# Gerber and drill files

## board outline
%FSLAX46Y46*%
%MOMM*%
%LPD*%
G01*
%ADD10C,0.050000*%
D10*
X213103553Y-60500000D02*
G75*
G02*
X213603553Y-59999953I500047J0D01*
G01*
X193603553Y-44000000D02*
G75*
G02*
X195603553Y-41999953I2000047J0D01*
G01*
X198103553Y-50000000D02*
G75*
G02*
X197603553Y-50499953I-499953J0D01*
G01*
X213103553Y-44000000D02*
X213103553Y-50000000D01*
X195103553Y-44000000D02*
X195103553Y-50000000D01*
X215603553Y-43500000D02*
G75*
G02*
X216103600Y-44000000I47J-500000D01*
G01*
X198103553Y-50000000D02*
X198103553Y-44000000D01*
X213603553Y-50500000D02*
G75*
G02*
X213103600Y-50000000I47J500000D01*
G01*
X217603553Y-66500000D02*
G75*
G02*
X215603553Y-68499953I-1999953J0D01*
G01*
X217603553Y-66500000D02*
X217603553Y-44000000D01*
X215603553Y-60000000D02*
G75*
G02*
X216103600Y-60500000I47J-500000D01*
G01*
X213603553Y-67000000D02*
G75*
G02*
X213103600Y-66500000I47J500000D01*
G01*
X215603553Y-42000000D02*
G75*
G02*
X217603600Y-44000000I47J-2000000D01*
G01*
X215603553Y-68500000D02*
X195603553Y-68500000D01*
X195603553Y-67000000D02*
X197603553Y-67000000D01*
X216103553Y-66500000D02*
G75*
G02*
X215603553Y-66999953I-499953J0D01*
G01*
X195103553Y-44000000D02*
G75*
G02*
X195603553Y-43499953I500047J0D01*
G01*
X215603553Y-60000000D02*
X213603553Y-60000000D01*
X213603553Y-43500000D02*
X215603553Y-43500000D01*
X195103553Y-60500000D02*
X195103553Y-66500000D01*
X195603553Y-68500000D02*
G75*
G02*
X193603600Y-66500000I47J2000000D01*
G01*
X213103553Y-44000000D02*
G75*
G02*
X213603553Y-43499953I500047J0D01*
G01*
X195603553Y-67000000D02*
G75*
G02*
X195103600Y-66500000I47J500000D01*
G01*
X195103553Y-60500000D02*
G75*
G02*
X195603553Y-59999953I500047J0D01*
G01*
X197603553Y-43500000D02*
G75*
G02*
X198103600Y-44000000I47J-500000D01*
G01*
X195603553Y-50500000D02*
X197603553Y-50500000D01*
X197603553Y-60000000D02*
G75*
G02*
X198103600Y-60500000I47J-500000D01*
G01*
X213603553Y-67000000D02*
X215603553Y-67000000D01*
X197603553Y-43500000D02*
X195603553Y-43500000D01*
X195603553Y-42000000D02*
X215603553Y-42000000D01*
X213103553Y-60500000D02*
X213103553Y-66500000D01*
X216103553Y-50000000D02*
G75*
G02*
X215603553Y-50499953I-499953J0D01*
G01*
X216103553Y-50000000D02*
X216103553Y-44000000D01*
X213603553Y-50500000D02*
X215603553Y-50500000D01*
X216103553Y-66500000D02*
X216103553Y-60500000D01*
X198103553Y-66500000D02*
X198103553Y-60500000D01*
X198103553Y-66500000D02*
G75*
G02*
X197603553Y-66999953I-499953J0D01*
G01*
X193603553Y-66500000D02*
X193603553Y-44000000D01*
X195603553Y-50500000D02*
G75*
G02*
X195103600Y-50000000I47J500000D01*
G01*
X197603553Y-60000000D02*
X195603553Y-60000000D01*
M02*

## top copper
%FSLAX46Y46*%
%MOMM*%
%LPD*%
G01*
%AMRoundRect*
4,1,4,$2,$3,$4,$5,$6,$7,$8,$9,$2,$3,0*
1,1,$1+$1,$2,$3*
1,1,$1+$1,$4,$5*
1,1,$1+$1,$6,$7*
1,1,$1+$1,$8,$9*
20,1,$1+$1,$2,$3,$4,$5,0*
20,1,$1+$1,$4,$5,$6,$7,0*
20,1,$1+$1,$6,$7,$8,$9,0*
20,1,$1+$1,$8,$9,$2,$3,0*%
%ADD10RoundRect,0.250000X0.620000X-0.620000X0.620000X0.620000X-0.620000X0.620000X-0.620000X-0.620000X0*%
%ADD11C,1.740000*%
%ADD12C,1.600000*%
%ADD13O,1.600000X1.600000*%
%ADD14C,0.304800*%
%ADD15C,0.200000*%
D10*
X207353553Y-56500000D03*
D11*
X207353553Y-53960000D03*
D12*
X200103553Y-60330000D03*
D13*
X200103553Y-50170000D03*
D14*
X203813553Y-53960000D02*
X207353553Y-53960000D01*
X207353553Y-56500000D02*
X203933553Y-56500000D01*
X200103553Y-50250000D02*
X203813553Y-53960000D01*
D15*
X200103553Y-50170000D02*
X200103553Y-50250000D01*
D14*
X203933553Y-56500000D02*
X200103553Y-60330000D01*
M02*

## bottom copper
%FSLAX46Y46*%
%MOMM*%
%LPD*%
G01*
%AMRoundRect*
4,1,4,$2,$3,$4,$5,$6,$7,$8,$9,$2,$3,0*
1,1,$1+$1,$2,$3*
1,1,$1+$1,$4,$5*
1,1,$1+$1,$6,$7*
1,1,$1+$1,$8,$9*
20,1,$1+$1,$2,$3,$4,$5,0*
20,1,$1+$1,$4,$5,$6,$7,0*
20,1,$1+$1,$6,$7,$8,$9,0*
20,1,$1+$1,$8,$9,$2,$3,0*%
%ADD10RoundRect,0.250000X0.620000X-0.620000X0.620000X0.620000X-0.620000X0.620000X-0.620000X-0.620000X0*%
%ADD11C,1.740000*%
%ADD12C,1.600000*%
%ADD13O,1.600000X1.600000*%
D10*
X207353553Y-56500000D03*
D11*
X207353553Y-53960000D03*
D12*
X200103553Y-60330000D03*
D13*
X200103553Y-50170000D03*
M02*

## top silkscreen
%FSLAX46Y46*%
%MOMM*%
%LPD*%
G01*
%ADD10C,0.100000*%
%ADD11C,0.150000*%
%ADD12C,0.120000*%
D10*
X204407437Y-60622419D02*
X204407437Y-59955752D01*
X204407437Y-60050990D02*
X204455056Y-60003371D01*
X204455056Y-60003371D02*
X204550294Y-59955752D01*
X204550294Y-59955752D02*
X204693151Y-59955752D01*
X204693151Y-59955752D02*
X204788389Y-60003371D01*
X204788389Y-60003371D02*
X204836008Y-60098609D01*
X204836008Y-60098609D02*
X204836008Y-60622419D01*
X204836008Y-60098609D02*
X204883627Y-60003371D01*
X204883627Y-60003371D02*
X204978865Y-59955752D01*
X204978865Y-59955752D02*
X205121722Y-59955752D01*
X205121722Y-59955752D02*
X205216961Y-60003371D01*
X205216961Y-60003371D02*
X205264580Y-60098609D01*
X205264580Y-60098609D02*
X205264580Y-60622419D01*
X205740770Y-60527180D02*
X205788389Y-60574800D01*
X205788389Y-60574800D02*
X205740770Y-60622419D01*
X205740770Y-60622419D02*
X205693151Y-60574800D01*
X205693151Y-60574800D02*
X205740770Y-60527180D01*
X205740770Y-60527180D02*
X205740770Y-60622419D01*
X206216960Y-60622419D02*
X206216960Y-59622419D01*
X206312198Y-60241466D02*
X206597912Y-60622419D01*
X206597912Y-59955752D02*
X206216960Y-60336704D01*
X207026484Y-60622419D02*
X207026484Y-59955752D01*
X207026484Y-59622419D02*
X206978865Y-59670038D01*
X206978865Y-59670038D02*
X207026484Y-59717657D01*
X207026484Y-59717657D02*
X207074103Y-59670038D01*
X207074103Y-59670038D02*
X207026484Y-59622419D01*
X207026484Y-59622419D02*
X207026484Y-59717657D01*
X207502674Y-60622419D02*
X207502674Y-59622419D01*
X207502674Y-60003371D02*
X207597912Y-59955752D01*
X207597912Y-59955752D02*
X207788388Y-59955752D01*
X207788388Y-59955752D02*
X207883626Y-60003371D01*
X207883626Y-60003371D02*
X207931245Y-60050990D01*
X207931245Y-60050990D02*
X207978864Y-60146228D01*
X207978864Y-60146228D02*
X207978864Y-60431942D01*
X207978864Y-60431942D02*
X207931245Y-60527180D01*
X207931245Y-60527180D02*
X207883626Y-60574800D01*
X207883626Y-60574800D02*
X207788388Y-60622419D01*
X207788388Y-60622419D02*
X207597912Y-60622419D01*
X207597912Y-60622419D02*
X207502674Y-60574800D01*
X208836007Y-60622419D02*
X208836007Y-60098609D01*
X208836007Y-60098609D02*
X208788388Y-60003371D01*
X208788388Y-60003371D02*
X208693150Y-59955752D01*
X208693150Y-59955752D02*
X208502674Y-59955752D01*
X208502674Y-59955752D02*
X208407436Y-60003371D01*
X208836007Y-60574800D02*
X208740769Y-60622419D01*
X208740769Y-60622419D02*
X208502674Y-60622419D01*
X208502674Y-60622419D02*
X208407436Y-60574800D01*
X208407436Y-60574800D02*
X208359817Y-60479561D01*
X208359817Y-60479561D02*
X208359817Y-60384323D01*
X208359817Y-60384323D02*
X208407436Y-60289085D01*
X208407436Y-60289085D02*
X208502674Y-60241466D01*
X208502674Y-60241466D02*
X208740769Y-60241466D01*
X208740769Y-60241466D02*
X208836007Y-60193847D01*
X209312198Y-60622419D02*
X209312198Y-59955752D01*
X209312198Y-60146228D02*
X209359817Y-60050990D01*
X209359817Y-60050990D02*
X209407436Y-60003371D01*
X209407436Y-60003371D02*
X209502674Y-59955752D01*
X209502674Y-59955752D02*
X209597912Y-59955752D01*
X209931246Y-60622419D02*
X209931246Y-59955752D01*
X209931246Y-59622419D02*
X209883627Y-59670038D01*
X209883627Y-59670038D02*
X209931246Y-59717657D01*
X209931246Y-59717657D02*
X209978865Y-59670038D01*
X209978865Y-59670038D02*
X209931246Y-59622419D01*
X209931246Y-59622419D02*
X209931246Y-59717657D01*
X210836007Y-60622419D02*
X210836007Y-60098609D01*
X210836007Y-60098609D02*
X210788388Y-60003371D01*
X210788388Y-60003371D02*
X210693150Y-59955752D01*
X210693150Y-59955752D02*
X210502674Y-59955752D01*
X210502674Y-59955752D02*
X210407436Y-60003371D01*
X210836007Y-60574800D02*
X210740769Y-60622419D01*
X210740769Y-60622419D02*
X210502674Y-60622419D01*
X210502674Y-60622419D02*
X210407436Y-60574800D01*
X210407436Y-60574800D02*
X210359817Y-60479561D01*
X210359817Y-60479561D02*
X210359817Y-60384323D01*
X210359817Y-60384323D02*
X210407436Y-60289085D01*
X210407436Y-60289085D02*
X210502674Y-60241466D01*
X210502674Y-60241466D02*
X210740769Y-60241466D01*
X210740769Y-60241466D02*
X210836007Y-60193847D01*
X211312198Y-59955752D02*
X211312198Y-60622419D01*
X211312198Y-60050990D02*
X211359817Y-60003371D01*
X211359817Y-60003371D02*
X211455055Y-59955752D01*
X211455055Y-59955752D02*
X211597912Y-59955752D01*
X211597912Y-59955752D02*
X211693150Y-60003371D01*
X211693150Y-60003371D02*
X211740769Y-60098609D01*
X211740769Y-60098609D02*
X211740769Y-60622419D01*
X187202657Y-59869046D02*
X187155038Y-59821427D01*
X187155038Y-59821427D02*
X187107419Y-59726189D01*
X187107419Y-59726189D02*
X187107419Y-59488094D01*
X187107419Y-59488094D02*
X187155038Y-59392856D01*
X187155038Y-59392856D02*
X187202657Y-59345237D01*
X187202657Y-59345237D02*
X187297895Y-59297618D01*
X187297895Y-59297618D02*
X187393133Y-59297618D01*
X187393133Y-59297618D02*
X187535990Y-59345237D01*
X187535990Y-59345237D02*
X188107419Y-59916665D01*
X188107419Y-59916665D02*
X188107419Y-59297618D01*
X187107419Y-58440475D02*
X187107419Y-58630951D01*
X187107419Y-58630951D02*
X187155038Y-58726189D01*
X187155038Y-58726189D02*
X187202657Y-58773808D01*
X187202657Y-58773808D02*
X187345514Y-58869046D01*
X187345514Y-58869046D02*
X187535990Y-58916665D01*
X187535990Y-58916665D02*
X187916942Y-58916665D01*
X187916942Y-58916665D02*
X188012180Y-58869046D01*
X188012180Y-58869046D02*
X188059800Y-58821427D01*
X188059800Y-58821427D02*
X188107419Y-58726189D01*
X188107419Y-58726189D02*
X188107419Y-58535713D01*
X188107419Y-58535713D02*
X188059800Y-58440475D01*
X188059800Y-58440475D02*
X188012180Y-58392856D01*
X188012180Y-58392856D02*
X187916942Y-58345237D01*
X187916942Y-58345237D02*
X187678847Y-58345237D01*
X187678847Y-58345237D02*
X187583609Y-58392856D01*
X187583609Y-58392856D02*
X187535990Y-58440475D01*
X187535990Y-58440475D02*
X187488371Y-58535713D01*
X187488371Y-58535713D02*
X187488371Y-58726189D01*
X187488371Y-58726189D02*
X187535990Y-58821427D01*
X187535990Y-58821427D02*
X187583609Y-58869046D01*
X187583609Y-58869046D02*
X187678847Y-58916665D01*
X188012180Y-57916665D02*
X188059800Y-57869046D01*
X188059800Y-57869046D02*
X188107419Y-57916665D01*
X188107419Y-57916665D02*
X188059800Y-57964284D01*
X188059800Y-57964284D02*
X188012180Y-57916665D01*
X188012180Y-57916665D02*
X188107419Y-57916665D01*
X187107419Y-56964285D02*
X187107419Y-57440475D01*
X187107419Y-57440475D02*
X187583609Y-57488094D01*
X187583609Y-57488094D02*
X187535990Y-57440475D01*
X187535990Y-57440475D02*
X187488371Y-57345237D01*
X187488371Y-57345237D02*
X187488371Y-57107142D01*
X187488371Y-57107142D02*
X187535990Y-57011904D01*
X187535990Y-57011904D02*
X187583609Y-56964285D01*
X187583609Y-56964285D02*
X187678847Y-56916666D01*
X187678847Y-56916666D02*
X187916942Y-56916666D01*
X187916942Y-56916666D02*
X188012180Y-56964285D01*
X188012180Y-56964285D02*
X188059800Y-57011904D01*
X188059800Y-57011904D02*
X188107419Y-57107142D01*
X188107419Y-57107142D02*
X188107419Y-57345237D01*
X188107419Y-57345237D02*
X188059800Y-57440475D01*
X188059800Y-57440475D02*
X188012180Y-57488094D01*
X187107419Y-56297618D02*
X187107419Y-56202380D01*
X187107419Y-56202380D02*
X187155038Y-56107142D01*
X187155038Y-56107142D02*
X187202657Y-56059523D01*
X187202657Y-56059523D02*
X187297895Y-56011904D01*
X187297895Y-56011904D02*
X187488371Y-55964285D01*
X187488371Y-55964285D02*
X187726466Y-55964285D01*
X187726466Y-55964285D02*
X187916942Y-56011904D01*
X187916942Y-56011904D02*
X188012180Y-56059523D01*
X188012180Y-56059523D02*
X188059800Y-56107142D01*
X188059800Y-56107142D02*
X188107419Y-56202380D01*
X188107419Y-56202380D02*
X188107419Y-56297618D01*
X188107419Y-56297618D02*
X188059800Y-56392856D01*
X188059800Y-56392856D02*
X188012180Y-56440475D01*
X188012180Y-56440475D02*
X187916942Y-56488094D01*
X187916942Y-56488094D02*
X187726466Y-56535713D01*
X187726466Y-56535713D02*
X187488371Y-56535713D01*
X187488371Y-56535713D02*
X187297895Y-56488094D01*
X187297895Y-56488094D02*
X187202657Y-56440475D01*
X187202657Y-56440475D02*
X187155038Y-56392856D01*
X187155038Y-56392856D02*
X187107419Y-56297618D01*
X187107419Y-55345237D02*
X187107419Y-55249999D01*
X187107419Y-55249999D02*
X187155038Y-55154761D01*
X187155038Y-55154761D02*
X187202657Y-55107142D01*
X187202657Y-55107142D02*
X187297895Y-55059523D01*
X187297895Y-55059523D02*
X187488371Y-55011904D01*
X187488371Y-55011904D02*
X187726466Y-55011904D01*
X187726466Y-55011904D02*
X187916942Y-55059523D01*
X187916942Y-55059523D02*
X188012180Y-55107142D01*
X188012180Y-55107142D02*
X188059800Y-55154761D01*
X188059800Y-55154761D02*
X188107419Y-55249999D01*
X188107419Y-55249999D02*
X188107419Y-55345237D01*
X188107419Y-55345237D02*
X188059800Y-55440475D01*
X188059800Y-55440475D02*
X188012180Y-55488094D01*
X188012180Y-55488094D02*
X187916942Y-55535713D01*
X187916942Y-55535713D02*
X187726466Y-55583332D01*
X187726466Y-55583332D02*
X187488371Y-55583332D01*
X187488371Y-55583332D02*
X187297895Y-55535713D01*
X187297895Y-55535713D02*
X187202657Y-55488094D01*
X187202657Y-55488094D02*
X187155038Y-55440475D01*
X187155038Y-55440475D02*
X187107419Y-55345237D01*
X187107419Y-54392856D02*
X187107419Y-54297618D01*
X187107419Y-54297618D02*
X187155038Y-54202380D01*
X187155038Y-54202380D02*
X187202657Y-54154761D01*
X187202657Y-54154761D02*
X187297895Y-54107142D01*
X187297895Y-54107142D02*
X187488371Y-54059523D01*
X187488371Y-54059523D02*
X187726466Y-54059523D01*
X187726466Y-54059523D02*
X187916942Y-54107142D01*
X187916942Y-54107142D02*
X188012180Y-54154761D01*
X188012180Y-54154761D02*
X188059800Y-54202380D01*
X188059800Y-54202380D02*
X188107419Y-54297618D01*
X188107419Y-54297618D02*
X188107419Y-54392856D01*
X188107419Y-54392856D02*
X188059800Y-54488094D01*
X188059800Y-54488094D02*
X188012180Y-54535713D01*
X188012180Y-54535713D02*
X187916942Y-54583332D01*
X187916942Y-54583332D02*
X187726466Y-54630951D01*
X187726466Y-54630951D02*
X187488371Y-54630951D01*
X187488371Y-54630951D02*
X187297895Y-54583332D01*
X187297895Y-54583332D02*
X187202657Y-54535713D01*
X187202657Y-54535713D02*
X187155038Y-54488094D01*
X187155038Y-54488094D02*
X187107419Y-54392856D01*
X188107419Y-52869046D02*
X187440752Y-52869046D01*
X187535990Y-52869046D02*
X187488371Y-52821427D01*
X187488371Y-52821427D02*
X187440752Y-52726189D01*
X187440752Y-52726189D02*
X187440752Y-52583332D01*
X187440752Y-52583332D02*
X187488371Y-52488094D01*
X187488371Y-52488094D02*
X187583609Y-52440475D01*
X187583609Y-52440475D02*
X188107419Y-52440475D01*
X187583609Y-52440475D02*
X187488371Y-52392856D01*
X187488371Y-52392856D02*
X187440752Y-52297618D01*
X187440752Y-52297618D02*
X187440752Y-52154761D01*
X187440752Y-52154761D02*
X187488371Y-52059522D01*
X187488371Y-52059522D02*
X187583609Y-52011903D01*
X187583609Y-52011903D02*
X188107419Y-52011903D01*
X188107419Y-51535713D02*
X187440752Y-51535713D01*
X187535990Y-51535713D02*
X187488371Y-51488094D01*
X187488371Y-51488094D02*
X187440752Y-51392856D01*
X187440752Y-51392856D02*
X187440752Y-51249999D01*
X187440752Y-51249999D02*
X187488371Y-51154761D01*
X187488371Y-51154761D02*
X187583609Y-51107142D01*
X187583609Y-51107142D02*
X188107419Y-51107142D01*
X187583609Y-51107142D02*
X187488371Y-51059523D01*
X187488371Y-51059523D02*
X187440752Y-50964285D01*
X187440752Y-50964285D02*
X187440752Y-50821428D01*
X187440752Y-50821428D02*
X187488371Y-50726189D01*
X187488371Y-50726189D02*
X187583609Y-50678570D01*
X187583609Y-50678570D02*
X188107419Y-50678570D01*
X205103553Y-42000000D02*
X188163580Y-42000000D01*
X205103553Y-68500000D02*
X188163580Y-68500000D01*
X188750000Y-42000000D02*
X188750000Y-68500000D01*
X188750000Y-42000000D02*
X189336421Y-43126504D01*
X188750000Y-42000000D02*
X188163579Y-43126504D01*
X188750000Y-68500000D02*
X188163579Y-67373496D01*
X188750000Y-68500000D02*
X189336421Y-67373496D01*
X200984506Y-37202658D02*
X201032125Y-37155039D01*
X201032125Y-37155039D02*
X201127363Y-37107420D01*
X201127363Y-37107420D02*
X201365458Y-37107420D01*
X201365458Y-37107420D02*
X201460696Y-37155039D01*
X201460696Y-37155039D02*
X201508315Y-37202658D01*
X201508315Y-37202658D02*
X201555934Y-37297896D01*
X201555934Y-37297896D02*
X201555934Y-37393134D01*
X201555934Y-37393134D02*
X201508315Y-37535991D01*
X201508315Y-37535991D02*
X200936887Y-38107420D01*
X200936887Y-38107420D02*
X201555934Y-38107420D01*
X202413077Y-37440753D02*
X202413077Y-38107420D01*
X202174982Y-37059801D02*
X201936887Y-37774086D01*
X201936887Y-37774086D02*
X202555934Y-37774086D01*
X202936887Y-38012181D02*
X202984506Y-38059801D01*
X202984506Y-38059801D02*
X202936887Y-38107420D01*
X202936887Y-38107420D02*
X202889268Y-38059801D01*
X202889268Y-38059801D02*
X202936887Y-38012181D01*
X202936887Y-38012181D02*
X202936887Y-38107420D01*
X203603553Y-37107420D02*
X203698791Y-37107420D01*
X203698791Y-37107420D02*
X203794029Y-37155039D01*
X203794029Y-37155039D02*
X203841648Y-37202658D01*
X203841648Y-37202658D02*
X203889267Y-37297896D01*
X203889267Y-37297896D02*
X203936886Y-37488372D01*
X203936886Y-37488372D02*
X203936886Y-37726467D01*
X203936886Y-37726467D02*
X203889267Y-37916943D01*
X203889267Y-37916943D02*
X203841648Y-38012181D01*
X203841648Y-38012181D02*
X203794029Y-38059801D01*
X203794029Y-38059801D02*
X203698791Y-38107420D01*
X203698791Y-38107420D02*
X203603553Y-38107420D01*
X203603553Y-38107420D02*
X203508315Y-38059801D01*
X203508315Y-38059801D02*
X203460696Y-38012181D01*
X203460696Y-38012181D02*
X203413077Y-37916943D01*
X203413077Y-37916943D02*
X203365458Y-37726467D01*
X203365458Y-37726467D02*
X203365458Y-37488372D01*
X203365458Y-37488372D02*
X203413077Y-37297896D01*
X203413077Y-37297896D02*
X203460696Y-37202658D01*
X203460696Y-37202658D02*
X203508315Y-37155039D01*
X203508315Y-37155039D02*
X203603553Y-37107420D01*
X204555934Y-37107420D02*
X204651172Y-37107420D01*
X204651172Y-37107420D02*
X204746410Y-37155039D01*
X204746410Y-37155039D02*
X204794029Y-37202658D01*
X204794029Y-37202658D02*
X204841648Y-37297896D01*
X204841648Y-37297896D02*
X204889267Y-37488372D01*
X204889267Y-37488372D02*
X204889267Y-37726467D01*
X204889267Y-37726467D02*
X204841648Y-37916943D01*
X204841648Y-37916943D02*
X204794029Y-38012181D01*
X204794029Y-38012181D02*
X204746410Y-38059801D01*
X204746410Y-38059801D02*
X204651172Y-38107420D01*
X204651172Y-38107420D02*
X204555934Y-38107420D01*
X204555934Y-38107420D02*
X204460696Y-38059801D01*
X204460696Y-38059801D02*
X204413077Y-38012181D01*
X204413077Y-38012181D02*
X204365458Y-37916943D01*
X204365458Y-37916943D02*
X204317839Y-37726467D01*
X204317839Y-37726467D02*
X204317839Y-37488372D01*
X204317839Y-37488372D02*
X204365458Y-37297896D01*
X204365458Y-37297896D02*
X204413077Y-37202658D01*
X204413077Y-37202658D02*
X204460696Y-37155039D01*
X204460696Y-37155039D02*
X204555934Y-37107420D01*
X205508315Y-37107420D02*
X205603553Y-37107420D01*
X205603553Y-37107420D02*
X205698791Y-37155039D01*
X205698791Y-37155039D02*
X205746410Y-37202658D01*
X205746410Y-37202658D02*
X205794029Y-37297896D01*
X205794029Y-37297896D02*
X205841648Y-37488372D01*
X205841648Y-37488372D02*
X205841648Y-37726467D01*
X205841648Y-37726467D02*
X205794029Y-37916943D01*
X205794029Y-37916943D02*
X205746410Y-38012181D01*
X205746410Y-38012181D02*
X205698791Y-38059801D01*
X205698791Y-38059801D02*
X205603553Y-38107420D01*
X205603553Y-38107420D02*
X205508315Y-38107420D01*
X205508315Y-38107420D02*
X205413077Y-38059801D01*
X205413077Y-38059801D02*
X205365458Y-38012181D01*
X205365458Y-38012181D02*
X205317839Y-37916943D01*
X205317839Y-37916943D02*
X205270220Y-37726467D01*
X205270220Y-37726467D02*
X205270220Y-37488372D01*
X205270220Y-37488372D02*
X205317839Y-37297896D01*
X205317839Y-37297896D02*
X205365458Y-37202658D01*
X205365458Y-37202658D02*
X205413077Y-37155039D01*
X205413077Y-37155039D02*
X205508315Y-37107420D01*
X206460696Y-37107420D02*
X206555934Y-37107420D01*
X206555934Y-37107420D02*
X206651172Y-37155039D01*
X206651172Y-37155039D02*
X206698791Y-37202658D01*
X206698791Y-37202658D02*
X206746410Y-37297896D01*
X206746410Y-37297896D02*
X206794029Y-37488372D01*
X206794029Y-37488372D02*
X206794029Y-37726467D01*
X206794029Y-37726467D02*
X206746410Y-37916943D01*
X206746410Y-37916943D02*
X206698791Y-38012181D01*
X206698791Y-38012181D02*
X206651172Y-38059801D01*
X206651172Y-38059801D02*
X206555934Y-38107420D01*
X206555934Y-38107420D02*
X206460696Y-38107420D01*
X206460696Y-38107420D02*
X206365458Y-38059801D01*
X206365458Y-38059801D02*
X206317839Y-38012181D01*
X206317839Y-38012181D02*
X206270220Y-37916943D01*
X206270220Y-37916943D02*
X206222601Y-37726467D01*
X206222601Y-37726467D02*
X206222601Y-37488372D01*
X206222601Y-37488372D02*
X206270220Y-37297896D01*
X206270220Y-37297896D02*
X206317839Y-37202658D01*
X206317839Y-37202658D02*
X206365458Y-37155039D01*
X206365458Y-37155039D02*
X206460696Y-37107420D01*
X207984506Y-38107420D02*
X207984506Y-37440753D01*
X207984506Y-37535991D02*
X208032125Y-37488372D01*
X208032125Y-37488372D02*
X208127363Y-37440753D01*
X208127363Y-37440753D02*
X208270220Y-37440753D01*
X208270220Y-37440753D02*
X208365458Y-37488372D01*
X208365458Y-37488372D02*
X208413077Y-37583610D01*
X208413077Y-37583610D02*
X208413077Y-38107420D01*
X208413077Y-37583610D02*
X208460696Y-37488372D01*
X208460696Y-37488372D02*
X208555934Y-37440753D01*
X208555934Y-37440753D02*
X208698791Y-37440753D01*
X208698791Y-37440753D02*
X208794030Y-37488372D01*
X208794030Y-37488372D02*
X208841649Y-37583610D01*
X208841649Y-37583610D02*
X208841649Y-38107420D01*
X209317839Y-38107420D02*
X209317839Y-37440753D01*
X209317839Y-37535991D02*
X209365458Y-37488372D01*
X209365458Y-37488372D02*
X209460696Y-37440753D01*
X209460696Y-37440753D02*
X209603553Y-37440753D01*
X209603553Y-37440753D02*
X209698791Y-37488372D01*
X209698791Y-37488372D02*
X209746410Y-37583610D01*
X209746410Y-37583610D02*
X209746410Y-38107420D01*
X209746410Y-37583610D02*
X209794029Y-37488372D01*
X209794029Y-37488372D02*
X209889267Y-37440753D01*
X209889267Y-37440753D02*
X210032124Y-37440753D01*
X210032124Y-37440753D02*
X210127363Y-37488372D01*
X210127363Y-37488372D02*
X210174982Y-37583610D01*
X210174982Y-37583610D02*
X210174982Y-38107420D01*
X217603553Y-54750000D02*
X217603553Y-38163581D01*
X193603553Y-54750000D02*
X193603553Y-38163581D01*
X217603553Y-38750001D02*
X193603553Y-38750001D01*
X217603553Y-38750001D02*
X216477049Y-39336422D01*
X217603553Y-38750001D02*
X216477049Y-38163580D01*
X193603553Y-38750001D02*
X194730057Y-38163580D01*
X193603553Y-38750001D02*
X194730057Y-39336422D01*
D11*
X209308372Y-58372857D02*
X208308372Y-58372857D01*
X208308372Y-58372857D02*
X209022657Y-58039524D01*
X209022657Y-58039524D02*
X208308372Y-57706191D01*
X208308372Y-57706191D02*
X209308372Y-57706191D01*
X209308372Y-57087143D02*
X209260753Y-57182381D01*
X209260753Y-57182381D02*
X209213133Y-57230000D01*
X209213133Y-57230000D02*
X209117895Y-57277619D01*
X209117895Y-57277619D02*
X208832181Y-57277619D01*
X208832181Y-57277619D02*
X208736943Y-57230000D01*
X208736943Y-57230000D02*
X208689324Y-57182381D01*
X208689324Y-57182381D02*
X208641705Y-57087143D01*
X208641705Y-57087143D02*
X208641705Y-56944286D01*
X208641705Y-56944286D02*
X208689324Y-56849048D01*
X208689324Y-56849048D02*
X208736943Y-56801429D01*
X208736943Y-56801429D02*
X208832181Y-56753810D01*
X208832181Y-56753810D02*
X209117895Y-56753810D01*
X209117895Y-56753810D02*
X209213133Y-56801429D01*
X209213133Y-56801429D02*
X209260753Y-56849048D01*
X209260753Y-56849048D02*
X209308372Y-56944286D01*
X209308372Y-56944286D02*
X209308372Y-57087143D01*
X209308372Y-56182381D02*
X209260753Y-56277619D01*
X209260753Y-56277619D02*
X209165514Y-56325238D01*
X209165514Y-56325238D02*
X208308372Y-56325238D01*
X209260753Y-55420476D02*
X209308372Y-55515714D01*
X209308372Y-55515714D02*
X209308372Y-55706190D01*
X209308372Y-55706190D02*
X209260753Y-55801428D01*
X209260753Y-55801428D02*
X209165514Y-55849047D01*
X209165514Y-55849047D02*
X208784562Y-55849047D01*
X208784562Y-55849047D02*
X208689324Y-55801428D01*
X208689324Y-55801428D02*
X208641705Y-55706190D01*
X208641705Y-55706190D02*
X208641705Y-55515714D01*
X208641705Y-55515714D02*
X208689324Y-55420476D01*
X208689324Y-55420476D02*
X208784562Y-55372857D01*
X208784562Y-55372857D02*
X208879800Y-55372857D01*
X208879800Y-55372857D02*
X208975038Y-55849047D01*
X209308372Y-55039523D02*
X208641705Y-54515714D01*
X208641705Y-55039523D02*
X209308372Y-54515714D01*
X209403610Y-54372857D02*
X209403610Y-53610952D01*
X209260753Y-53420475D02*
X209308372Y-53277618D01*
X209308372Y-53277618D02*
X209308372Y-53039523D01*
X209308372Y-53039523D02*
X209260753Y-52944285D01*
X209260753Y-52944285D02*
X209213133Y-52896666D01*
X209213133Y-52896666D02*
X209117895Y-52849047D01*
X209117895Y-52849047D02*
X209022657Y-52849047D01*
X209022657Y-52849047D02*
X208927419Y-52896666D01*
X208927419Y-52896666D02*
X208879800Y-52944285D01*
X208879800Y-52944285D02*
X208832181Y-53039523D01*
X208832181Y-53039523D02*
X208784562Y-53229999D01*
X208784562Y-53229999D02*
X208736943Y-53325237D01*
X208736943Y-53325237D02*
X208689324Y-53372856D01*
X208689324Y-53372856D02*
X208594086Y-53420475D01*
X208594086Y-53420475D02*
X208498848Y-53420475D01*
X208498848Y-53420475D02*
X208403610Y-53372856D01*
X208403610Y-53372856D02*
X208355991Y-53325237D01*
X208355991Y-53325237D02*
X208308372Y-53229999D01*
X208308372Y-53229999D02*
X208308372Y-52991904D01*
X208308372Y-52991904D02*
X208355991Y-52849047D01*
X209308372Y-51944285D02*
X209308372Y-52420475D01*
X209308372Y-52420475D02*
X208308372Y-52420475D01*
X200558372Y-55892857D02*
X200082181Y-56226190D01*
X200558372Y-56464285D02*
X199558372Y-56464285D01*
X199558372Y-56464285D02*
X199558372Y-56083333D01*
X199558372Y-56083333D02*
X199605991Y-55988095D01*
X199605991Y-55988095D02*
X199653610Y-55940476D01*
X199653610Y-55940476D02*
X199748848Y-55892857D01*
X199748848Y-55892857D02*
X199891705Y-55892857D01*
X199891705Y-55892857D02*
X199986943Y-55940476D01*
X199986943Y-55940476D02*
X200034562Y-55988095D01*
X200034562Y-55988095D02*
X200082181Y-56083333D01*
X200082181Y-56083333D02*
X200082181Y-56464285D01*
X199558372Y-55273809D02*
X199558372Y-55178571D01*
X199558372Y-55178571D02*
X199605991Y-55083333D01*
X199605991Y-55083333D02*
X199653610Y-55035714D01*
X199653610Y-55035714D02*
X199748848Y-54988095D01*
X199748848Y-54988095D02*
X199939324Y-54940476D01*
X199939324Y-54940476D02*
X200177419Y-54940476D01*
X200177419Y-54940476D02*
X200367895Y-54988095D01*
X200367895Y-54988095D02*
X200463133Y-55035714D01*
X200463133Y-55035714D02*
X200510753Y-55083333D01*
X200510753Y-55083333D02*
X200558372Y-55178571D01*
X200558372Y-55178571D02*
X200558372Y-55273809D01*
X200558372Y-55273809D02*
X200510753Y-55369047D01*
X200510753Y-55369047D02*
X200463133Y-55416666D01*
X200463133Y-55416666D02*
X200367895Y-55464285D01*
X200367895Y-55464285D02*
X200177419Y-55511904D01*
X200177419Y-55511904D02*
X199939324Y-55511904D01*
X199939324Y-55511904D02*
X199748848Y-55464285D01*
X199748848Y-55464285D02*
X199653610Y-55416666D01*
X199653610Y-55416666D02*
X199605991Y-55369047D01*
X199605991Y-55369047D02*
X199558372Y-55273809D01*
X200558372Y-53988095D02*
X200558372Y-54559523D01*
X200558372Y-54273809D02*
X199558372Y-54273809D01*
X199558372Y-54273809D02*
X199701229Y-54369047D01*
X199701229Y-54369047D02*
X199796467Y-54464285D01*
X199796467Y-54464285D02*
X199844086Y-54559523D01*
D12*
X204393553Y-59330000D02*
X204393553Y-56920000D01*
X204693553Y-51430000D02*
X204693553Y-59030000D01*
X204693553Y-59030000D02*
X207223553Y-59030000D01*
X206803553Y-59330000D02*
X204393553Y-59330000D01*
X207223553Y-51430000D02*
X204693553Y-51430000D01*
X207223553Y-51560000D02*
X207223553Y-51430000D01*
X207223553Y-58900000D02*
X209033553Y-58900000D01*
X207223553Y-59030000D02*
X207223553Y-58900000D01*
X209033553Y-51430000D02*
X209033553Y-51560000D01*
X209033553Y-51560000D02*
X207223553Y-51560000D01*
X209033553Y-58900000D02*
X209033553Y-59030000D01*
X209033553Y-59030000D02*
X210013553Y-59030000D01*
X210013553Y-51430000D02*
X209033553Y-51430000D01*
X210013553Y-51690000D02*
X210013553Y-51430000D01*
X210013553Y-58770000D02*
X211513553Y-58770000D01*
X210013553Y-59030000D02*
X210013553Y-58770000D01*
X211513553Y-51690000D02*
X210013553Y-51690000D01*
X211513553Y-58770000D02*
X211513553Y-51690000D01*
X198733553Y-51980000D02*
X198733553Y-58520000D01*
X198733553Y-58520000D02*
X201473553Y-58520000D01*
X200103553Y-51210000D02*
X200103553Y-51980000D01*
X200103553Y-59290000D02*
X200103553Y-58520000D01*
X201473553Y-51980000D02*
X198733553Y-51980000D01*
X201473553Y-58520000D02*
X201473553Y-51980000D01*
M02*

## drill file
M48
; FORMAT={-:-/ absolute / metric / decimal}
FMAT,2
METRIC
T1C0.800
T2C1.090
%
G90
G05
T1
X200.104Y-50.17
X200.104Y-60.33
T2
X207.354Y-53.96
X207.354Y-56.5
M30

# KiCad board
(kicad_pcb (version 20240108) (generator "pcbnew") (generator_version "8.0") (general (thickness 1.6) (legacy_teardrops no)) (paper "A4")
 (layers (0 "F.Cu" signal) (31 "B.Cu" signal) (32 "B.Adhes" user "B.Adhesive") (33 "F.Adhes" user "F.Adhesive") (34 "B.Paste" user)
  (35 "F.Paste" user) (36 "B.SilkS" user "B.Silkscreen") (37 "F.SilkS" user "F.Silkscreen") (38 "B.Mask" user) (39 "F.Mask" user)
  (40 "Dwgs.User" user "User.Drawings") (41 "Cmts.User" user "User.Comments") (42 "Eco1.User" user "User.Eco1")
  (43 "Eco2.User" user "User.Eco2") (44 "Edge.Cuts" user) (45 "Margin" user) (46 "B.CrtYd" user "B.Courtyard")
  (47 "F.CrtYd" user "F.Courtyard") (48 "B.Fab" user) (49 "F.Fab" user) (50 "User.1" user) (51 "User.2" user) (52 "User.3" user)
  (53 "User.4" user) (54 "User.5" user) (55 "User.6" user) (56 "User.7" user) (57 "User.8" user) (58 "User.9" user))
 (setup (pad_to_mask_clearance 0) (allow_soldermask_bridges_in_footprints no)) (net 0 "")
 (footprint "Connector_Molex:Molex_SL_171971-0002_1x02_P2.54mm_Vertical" (layer "F.Cu") (at 207.353553 56.5 90)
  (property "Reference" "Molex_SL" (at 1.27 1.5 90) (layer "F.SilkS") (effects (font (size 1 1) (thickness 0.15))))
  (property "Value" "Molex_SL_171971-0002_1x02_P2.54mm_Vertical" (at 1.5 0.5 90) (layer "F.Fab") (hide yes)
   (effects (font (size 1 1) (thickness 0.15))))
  (fp_line (start -2.83 -2.96) (end -0.42 -2.96) (stroke (width 0.12) (type solid)) (layer "F.SilkS"))
  (fp_line (start 5.07 -2.66) (end -2.53 -2.66) (stroke (width 0.12) (type solid)) (layer "F.SilkS"))
  (fp_line (start -2.53 -2.66) (end -2.53 -0.13) (stroke (width 0.12) (type solid)) (layer "F.SilkS"))
  (fp_line (start -2.83 -0.55) (end -2.83 -2.96) (stroke (width 0.12) (type solid)) (layer "F.SilkS"))
  (fp_line (start 5.07 -0.13) (end 5.07 -2.66) (stroke (width 0.12) (type solid)) (layer "F.SilkS"))
  (fp_line (start 4.94 -0.13) (end 5.07 -0.13) (stroke (width 0.12) (type solid)) (layer "F.SilkS"))
  (fp_line (start -2.4 -0.13) (end -2.4 1.68) (stroke (width 0.12) (type solid)) (layer "F.SilkS"))
  (fp_line (start -2.53 -0.13) (end -2.4 -0.13) (stroke (width 0.12) (type solid)) (layer "F.SilkS"))
  (fp_line (start 5.07 1.68) (end 4.94 1.68) (stroke (width 0.12) (type solid)) (layer "F.SilkS"))
  (fp_line (start 4.94 1.68) (end 4.94 -0.13) (stroke (width 0.12) (type solid)) (layer "F.SilkS"))
  (fp_line (start -2.4 1.68) (end -2.53 1.68) (stroke (width 0.12) (type solid)) (layer "F.SilkS"))
  (fp_line (start -2.53 1.68) (end -2.53 2.66) (stroke (width 0.12) (type solid)) (layer "F.SilkS"))
  (fp_line (start 5.07 2.66) (end 5.07 1.68) (stroke (width 0.12) (type solid)) (layer "F.SilkS"))
  (fp_line (start 4.81 2.66) (end 5.07 2.66) (stroke (width 0.12) (type solid)) (layer "F.SilkS"))
  (fp_line (start -2.27 2.66) (end -2.27 4.16) (stroke (width 0.12) (type solid)) (layer "F.SilkS"))
  (fp_line (start -2.53 2.66) (end -2.27 2.66) (stroke (width 0.12) (type solid)) (layer "F.SilkS"))
  (fp_line (start 4.81 4.16) (end 4.81 2.66) (stroke (width 0.12) (type solid)) (layer "F.SilkS"))
  (fp_line (start -2.27 4.16) (end 4.81 4.16) (stroke (width 0.12) (type solid)) (layer "F.SilkS"))
  (pad "1" thru_hole roundrect (at 0 0 90) (size 1.74 1.74) (drill 1.09) (layers "*.Cu" "*.Mask") (remove_unused_layers no)
   (roundrect_rratio 0.143678))
  (pad "2" thru_hole circle (at 2.54 0 90) (size 1.74 1.74) (drill 1.09) (layers "*.Cu" "*.Mask") (remove_unused_layers no)))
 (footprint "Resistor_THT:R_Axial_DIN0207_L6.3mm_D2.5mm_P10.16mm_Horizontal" (layer "F.Cu") (at 200.103553 60.33 90)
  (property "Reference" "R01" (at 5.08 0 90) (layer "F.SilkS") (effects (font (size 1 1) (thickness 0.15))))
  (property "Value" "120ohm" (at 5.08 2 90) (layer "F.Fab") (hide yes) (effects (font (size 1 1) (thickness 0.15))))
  (fp_line (start 8.35 -1.37) (end 1.81 -1.37) (stroke (width 0.12) (type solid)) (layer "F.SilkS"))
  (fp_line (start 1.81 -1.37) (end 1.81 1.37) (stroke (width 0.12) (type solid)) (layer "F.SilkS"))
  (fp_line (start 9.12 0) (end 8.35 0) (stroke (width 0.12) (type solid)) (layer "F.SilkS"))
  (fp_line (start 1.04 0) (end 1.81 0) (stroke (width 0.12) (type solid)) (layer "F.SilkS"))
  (fp_line (start 8.35 1.37) (end 8.35 -1.37) (stroke (width 0.12) (type solid)) (layer "F.SilkS"))
  (fp_line (start 1.81 1.37) (end 8.35 1.37) (stroke (width 0.12) (type solid)) (layer "F.SilkS"))
  (pad "1" thru_hole circle (at 0 0 90) (size 1.6 1.6) (drill 0.8) (layers "*.Cu" "*.Mask") (remove_unused_layers no))
  (pad "2" thru_hole oval (at 10.16 0 90) (size 1.6 1.6) (drill 0.8) (layers "*.Cu" "*.Mask") (remove_unused_layers no)))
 (gr_arc (start 213.103553 60.5) (mid 213.25 60.146447) (end 213.603553 60) (stroke (width 0.05) (type default)) (layer "Edge.Cuts"))
 (gr_arc (start 193.603553 44) (mid 194.189339 42.585786) (end 195.603553 42) (stroke (width 0.05) (type default)) (layer "Edge.Cuts"))
 (gr_arc (start 198.103553 50) (mid 197.957106 50.353553) (end 197.603553 50.5) (stroke (width 0.05) (type default)) (layer "Edge.Cuts"))
 (gr_line (start 213.103553 44) (end 213.103553 50) (stroke (width 0.05) (type default)) (layer "Edge.Cuts"))
 (gr_line (start 195.103553 44) (end 195.103553 50) (stroke (width 0.05) (type default)) (layer "Edge.Cuts"))
 (gr_arc (start 215.603553 43.5) (mid 215.957106 43.646447) (end 216.103553 44) (stroke (width 0.05) (type default)) (layer "Edge.Cuts"))
 (gr_line (start 198.103553 50) (end 198.103553 44) (stroke (width 0.05) (type default)) (layer "Edge.Cuts"))
 (gr_arc (start 213.603553 50.5) (mid 213.25 50.353553) (end 213.103553 50) (stroke (width 0.05) (type default)) (layer "Edge.Cuts"))
 (gr_arc (start 217.603553 66.5) (mid 217.017767 67.914214) (end 215.603553 68.5) (stroke (width 0.05) (type default)) (layer "Edge.Cuts"))
 (gr_line (start 217.603553 66.5) (end 217.603553 44) (stroke (width 0.05) (type default)) (layer "Edge.Cuts"))
 (gr_arc (start 215.603553 60) (mid 215.957106 60.146447) (end 216.103553 60.5) (stroke (width 0.05) (type default)) (layer "Edge.Cuts"))
 (gr_arc (start 213.603553 67) (mid 213.25 66.853553) (end 213.103553 66.5) (stroke (width 0.05) (type default)) (layer "Edge.Cuts"))
 (gr_arc (start 215.603553 42) (mid 217.017767 42.585786) (end 217.603553 44) (stroke (width 0.05) (type default)) (layer "Edge.Cuts"))
 (gr_line (start 215.603553 68.5) (end 195.603553 68.5) (stroke (width 0.05) (type default)) (layer "Edge.Cuts"))
 (gr_line (start 195.603553 67) (end 197.603553 67) (stroke (width 0.05) (type default)) (layer "Edge.Cuts"))
 (gr_arc (start 216.103553 66.5) (mid 215.957106 66.853553) (end 215.603553 67) (stroke (width 0.05) (type default)) (layer "Edge.Cuts"))
 (gr_arc (start 195.103553 44) (mid 195.25 43.646447) (end 195.603553 43.5) (stroke (width 0.05) (type default)) (layer "Edge.Cuts"))
 (gr_line (start 215.603553 60) (end 213.603553 60) (stroke (width 0.05) (type default)) (layer "Edge.Cuts"))
 (gr_line (start 213.603553 43.5) (end 215.603553 43.5) (stroke (width 0.05) (type default)) (layer "Edge.Cuts"))
 (gr_line (start 195.103553 60.5) (end 195.103553 66.5) (stroke (width 0.05) (type default)) (layer "Edge.Cuts"))
 (gr_arc (start 195.603553 68.5) (mid 194.189339 67.914214) (end 193.603553 66.5) (stroke (width 0.05) (type default)) (layer "Edge.Cuts"))
 (gr_arc (start 213.103553 44) (mid 213.25 43.646447) (end 213.603553 43.5) (stroke (width 0.05) (type default)) (layer "Edge.Cuts"))
 (gr_arc (start 195.603553 67) (mid 195.25 66.853553) (end 195.103553 66.5) (stroke (width 0.05) (type default)) (layer "Edge.Cuts"))
 (gr_arc (start 195.103553 60.5) (mid 195.25 60.146447) (end 195.603553 60) (stroke (width 0.05) (type default)) (layer "Edge.Cuts"))
 (gr_arc (start 197.603553 43.5) (mid 197.957106 43.646447) (end 198.103553 44) (stroke (width 0.05) (type default)) (layer "Edge.Cuts"))
 (gr_line (start 195.603553 50.5) (end 197.603553 50.5) (stroke (width 0.05) (type default)) (layer "Edge.Cuts"))
 (gr_arc (start 197.603553 60) (mid 197.957106 60.146447) (end 198.103553 60.5) (stroke (width 0.05) (type default)) (layer "Edge.Cuts"))
 (gr_line (start 213.603553 67) (end 215.603553 67) (stroke (width 0.05) (type default)) (layer "Edge.Cuts"))
 (gr_line (start 197.603553 43.5) (end 195.603553 43.5) (stroke (width 0.05) (type default)) (layer "Edge.Cuts"))
 (gr_line (start 195.603553 42) (end 215.603553 42) (stroke (width 0.05) (type default)) (layer "Edge.Cuts"))
 (gr_line (start 213.103553 60.5) (end 213.103553 66.5) (stroke (width 0.05) (type default)) (layer "Edge.Cuts"))
 (gr_arc (start 216.103553 50) (mid 215.957106 50.353553) (end 215.603553 50.5) (stroke (width 0.05) (type default)) (layer "Edge.Cuts"))
 (gr_line (start 216.103553 50) (end 216.103553 44) (stroke (width 0.05) (type default)) (layer "Edge.Cuts"))
 (gr_line (start 213.603553 50.5) (end 215.603553 50.5) (stroke (width 0.05) (type default)) (layer "Edge.Cuts"))
 (gr_line (start 216.103553 66.5) (end 216.103553 60.5) (stroke (width 0.05) (type default)) (layer "Edge.Cuts"))
 (gr_line (start 198.103553 66.5) (end 198.103553 60.5) (stroke (width 0.05) (type default)) (layer "Edge.Cuts"))
 (gr_arc (start 198.103553 66.5) (mid 197.957106 66.853553) (end 197.603553 67) (stroke (width 0.05) (type default)) (layer "Edge.Cuts"))
 (gr_line (start 193.603553 66.5) (end 193.603553 44) (stroke (width 0.05) (type default)) (layer "Edge.Cuts"))
 (gr_arc (start 195.603553 50.5) (mid 195.25 50.353553) (end 195.103553 50) (stroke (width 0.05) (type default)) (layer "Edge.Cuts"))
 (gr_line (start 197.603553 60) (end 195.603553 60) (stroke (width 0.05) (type default)) (layer "Edge.Cuts"))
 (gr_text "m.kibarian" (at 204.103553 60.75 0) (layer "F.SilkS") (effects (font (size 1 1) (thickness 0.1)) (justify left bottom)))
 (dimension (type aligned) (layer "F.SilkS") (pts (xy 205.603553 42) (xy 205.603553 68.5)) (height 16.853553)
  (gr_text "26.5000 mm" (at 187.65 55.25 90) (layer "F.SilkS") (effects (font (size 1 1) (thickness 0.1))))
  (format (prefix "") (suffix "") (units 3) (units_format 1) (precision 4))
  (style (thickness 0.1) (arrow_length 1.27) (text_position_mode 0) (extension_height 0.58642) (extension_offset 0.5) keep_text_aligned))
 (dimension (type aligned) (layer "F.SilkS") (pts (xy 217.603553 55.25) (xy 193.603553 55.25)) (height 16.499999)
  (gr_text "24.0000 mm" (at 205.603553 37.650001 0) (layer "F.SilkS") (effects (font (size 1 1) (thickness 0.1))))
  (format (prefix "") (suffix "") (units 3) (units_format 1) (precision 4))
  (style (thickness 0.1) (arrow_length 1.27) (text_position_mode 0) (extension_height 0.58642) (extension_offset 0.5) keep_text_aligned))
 (segment (start 203.813553 53.96) (end 207.353553 53.96) (width 0.3048) (layer "F.Cu") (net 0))
 (segment (start 207.353553 56.5) (end 203.933553 56.5) (width 0.3048) (layer "F.Cu") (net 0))
 (segment (start 200.103553 50.25) (end 203.813553 53.96) (width 0.3048) (layer "F.Cu") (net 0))
 (segment (start 200.103553 50.17) (end 200.103553 50.25) (width 0.2) (layer "F.Cu") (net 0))
 (segment (start 203.933553 56.5) (end 200.103553 60.33) (width 0.3048) (layer "F.Cu") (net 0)))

